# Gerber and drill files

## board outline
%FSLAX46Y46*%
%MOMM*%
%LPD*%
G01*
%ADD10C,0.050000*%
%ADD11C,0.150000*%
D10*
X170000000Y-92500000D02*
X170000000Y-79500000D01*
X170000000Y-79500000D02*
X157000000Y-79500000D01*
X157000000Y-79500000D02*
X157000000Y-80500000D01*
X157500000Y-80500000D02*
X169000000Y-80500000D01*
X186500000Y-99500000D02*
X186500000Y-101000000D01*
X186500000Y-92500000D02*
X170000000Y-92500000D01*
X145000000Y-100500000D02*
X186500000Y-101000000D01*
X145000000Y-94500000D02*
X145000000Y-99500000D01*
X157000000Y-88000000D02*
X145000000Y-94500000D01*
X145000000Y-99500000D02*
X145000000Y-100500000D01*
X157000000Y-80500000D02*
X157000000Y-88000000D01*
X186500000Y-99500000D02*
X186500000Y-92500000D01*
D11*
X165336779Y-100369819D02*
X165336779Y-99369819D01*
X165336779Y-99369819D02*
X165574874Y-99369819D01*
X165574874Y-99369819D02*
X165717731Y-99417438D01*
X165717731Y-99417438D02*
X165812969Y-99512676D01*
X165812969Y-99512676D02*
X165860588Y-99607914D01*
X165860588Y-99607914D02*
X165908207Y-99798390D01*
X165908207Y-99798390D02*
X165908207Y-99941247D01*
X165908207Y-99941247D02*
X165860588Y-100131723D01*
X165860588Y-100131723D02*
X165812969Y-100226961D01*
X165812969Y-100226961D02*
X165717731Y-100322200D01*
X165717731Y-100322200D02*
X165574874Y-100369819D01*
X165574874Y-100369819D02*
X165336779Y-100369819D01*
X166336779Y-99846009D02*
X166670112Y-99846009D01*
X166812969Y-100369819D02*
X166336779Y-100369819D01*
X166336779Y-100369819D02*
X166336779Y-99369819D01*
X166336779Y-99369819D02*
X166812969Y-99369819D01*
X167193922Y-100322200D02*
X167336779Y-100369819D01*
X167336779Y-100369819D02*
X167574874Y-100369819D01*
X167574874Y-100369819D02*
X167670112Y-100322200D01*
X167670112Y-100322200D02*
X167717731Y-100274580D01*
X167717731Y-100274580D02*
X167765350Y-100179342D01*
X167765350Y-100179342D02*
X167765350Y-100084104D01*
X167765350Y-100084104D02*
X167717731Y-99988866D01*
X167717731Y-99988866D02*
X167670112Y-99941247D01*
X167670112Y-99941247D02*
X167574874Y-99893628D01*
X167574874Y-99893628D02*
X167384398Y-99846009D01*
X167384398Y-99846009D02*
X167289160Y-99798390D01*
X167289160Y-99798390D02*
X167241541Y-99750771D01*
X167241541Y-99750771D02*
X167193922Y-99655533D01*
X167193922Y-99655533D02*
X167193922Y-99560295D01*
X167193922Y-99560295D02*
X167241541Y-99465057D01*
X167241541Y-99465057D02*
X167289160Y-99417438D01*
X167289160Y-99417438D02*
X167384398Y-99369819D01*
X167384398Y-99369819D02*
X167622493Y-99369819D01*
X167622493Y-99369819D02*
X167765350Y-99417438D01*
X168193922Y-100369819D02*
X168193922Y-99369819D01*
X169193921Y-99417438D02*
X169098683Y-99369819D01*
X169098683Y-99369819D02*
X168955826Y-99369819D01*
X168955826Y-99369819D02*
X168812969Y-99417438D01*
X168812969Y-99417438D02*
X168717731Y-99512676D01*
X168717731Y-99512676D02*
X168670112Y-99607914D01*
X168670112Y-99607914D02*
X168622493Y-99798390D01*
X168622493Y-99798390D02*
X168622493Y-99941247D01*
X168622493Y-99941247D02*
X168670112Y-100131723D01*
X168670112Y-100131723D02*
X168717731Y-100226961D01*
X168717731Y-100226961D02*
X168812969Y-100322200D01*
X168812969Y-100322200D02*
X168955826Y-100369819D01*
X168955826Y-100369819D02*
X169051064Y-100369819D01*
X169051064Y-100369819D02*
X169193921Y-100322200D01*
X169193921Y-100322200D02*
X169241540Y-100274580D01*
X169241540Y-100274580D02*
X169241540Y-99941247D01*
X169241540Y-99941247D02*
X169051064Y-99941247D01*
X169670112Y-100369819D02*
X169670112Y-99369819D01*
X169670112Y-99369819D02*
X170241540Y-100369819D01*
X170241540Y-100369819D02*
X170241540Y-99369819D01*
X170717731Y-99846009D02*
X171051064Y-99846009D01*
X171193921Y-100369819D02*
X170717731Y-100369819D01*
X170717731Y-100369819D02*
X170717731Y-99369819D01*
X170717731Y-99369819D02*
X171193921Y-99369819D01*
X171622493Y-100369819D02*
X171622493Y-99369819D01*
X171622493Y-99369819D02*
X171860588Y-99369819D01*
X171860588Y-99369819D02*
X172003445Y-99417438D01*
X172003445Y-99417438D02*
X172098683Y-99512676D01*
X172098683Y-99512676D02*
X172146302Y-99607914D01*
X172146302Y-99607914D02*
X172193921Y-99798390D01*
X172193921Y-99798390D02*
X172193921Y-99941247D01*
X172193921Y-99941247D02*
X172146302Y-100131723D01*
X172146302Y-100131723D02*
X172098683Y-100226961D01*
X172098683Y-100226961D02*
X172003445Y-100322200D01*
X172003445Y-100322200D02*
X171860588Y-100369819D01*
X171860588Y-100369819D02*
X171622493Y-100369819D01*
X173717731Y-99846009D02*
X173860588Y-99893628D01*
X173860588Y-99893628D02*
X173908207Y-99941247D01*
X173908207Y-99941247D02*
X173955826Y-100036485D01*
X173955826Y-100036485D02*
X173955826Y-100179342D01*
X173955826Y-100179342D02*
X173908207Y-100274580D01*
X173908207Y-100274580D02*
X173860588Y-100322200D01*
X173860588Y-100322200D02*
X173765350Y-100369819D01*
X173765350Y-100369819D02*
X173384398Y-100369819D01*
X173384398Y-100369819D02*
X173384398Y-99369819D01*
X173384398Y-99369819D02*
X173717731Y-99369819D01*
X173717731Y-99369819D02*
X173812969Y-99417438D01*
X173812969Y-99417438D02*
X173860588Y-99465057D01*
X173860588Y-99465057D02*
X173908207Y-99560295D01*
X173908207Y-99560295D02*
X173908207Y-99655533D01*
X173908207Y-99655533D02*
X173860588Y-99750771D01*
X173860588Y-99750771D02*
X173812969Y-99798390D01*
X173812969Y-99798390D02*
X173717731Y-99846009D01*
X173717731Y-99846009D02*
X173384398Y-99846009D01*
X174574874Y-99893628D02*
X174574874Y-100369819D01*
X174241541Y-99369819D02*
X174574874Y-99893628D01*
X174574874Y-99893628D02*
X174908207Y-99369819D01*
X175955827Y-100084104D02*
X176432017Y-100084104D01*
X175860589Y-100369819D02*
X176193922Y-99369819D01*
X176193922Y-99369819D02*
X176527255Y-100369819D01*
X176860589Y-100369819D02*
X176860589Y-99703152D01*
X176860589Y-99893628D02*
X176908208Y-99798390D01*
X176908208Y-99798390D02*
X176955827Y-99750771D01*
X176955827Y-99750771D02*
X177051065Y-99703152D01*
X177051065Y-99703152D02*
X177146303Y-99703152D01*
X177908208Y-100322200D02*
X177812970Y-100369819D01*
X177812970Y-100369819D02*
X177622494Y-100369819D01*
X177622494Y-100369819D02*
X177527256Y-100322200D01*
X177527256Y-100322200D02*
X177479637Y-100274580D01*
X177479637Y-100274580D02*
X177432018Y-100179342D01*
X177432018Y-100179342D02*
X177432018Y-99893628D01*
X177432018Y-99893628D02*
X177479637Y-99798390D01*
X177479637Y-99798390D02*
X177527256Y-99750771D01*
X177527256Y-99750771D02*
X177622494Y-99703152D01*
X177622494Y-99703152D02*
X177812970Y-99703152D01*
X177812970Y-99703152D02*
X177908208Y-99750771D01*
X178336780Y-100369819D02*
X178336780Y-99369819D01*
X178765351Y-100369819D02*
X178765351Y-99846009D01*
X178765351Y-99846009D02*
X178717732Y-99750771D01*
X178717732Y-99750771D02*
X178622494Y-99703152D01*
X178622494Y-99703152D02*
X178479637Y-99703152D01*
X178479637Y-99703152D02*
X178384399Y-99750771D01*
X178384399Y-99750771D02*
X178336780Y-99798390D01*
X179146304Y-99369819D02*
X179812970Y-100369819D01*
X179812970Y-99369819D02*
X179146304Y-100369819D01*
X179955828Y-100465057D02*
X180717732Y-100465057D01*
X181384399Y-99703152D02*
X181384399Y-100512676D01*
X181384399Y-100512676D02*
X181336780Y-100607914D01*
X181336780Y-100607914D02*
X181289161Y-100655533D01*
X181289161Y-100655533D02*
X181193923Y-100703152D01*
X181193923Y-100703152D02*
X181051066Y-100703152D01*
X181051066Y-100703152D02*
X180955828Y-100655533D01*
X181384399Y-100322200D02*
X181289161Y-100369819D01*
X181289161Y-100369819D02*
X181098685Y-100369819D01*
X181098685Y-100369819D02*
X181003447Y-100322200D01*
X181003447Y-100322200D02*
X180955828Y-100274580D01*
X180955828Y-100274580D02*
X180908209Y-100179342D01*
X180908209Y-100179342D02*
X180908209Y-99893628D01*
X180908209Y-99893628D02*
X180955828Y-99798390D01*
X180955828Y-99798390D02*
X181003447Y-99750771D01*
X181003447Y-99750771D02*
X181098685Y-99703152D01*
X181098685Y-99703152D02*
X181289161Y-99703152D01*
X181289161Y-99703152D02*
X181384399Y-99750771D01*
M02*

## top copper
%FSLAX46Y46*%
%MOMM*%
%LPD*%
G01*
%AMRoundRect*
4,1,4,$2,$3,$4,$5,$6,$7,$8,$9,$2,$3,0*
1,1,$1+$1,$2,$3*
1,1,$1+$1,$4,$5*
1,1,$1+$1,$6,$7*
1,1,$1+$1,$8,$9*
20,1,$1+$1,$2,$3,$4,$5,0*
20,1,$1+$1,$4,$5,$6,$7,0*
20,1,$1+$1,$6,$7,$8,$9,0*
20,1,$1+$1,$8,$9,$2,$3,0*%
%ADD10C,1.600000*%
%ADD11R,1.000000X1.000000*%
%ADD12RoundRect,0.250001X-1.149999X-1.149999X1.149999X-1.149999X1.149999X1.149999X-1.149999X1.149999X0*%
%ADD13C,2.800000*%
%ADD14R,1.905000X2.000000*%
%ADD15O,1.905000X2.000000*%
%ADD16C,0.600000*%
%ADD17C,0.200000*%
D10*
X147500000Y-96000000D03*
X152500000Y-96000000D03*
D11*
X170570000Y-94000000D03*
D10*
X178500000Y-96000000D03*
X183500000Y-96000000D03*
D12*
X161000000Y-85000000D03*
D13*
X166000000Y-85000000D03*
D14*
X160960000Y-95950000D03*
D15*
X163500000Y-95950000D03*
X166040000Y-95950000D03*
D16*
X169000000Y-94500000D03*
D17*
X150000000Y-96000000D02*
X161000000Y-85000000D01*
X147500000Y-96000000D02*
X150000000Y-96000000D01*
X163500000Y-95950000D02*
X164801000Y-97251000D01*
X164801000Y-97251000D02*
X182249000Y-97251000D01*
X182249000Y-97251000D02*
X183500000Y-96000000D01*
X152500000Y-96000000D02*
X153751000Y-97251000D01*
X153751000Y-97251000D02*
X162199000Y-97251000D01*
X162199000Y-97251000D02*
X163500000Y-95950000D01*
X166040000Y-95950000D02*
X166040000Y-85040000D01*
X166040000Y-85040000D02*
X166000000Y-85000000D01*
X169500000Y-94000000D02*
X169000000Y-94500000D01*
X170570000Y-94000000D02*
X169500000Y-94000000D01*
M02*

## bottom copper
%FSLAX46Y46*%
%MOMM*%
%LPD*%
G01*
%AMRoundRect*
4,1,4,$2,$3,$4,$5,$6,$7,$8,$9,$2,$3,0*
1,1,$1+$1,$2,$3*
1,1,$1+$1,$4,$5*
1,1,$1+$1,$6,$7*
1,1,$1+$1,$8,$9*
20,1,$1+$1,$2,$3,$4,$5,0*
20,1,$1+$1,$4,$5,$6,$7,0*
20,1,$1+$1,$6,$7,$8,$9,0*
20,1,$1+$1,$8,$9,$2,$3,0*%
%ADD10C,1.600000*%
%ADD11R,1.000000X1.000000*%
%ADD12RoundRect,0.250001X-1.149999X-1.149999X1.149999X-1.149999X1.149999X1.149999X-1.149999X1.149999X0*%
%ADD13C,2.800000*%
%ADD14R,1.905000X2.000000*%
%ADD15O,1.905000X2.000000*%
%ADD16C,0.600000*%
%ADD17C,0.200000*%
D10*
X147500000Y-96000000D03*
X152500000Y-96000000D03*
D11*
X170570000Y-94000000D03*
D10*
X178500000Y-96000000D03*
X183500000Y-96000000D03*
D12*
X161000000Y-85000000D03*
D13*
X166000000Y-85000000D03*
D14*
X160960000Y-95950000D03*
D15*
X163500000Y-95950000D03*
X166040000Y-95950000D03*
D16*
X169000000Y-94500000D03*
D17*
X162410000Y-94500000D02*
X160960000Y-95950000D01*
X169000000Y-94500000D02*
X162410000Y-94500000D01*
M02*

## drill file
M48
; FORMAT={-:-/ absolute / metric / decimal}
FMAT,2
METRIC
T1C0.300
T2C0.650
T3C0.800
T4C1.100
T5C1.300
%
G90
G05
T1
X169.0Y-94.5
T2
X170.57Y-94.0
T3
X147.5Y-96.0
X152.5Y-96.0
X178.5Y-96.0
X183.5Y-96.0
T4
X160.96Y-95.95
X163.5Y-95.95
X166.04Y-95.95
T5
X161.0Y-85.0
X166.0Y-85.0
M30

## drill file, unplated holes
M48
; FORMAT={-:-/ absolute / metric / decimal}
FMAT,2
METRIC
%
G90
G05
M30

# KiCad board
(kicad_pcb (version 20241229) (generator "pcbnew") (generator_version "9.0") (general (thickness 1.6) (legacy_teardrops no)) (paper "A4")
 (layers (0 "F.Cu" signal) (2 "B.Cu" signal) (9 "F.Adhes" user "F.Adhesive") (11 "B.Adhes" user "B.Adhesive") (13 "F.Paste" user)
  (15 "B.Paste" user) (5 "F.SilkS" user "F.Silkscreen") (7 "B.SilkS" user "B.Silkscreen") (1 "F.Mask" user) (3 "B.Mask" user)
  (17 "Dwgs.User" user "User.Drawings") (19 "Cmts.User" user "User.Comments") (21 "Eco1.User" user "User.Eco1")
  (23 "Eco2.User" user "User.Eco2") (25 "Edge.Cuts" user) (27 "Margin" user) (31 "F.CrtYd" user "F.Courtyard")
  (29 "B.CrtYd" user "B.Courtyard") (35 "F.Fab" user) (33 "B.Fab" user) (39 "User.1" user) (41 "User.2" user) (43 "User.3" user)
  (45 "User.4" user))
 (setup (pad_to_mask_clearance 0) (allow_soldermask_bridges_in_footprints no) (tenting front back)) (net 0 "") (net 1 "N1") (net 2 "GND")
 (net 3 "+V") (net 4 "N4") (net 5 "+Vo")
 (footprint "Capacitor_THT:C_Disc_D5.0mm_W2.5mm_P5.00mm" (layer "F.Cu") (at 147.5 96)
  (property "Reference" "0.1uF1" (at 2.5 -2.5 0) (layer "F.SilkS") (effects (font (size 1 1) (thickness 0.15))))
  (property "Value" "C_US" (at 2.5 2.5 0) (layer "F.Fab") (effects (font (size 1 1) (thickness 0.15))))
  (pad "1" thru_hole circle (at 0 0) (size 1.6 1.6) (drill 0.8) (layers "*.Cu" "*.Mask") (remove_unused_layers no) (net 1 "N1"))
  (pad "2" thru_hole circle (at 5 0) (size 1.6 1.6) (drill 0.8) (layers "*.Cu" "*.Mask") (remove_unused_layers no) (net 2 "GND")))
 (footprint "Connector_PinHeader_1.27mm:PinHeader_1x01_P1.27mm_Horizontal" (layer "F.Cu") (at 170.57 94)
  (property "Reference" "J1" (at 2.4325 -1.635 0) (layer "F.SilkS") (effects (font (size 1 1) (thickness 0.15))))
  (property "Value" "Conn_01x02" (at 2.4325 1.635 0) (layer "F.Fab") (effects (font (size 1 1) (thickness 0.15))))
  (pad "1" thru_hole rect (at 0 0) (size 1 1) (drill 0.65) (layers "*.Cu" "*.Mask") (remove_unused_layers no) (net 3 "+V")))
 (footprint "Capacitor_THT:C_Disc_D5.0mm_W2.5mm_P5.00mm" (layer "F.Cu") (at 178.5 96)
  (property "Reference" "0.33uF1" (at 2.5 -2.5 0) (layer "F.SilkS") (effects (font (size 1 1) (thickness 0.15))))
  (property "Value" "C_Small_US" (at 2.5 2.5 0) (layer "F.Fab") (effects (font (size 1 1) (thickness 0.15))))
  (pad "1" thru_hole circle (at 0 0) (size 1.6 1.6) (drill 0.8) (layers "*.Cu" "*.Mask") (remove_unused_layers no) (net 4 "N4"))
  (pad "2" thru_hole circle (at 5 0) (size 1.6 1.6) (drill 0.8) (layers "*.Cu" "*.Mask") (remove_unused_layers no) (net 2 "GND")))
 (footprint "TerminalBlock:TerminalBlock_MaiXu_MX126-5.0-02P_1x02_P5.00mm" (layer "F.Cu") (at 161 85)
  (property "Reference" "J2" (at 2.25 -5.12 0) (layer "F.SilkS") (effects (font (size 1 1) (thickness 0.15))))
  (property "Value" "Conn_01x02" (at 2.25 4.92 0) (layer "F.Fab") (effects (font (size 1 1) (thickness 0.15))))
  (pad "1" thru_hole roundrect (at 0 0) (size 2.8 2.8) (drill 1.3) (layers "*.Cu" "*.Mask") (remove_unused_layers no)
   (roundrect_rratio 0.089286) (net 1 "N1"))
  (pad "2" thru_hole circle (at 5 0) (size 2.8 2.8) (drill 1.3) (layers "*.Cu" "*.Mask") (remove_unused_layers no) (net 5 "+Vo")))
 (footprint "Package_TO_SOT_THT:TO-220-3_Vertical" (layer "F.Cu") (at 160.96 95.95)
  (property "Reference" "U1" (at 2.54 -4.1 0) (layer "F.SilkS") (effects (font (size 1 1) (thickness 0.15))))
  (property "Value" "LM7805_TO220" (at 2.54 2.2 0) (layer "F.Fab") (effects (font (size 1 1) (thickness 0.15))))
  (pad "1" thru_hole rect (at 0 0) (size 1.905 2) (drill 1.1) (layers "*.Cu" "*.Mask") (remove_unused_layers no) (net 3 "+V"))
  (pad "2" thru_hole oval (at 2.54 0) (size 1.905 2) (drill 1.1) (layers "*.Cu" "*.Mask") (remove_unused_layers no) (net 2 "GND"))
  (pad "3" thru_hole oval (at 5.08 0) (size 1.905 2) (drill 1.1) (layers "*.Cu" "*.Mask") (remove_unused_layers no) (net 5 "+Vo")))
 (gr_line (start 170 92.5) (end 170 79.5) (stroke (width 0.05) (type default)) (layer "Edge.Cuts"))
 (gr_line (start 170 79.5) (end 157 79.5) (stroke (width 0.05) (type default)) (layer "Edge.Cuts"))
 (gr_line (start 157 79.5) (end 157 80.5) (stroke (width 0.05) (type default)) (layer "Edge.Cuts"))
 (gr_line (start 157.5 80.5) (end 169 80.5) (stroke (width 0.05) (type default)) (layer "Edge.Cuts"))
 (gr_line (start 186.5 99.5) (end 186.5 101) (stroke (width 0.05) (type default)) (layer "Edge.Cuts"))
 (gr_line (start 186.5 92.5) (end 170 92.5) (stroke (width 0.05) (type default)) (layer "Edge.Cuts"))
 (gr_line (start 145 100.5) (end 186.5 101) (stroke (width 0.05) (type default)) (layer "Edge.Cuts"))
 (gr_line (start 145 94.5) (end 145 99.5) (stroke (width 0.05) (type default)) (layer "Edge.Cuts"))
 (gr_line (start 157 88) (end 145 94.5) (stroke (width 0.05) (type default)) (layer "Edge.Cuts"))
 (gr_line (start 145 99.5) (end 145 100.5) (stroke (width 0.05) (type default)) (layer "Edge.Cuts"))
 (gr_line (start 157 80.5) (end 157 88) (stroke (width 0.05) (type default)) (layer "Edge.Cuts"))
 (gr_line (start 186.5 99.5) (end 186.5 92.5) (stroke (width 0.05) (type default)) (layer "Edge.Cuts"))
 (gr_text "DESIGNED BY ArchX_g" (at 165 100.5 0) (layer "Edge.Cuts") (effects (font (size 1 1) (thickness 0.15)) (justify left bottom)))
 (segment (start 150 96) (end 161 85) (width 0.2) (layer "F.Cu") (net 1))
 (segment (start 147.5 96) (end 150 96) (width 0.2) (layer "F.Cu") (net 1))
 (segment (start 163.5 95.95) (end 164.801 97.251) (width 0.2) (layer "F.Cu") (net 2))
 (segment (start 164.801 97.251) (end 182.249 97.251) (width 0.2) (layer "F.Cu") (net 2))
 (segment (start 182.249 97.251) (end 183.5 96) (width 0.2) (layer "F.Cu") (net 2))
 (segment (start 152.5 96) (end 153.751 97.251) (width 0.2) (layer "F.Cu") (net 2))
 (segment (start 153.751 97.251) (end 162.199 97.251) (width 0.2) (layer "F.Cu") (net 2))
 (segment (start 162.199 97.251) (end 163.5 95.95) (width 0.2) (layer "F.Cu") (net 2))
 (segment (start 166.04 95.95) (end 166.04 85.04) (width 0.2) (layer "F.Cu") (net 5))
 (segment (start 166.04 85.04) (end 166 85) (width 0.2) (layer "F.Cu") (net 5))
 (segment (start 169.5 94) (end 169 94.5) (width 0.2) (layer "F.Cu") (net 3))
 (segment (start 170.57 94) (end 169.5 94) (width 0.2) (layer "F.Cu") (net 3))
 (via (at 169 94.5) (size 0.6) (drill 0.3) (layers "F.Cu" "B.Cu") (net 3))
 (segment (start 162.41 94.5) (end 160.96 95.95) (width 0.2) (layer "B.Cu") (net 3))
 (segment (start 169 94.5) (end 162.41 94.5) (width 0.2) (layer "B.Cu") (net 3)))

